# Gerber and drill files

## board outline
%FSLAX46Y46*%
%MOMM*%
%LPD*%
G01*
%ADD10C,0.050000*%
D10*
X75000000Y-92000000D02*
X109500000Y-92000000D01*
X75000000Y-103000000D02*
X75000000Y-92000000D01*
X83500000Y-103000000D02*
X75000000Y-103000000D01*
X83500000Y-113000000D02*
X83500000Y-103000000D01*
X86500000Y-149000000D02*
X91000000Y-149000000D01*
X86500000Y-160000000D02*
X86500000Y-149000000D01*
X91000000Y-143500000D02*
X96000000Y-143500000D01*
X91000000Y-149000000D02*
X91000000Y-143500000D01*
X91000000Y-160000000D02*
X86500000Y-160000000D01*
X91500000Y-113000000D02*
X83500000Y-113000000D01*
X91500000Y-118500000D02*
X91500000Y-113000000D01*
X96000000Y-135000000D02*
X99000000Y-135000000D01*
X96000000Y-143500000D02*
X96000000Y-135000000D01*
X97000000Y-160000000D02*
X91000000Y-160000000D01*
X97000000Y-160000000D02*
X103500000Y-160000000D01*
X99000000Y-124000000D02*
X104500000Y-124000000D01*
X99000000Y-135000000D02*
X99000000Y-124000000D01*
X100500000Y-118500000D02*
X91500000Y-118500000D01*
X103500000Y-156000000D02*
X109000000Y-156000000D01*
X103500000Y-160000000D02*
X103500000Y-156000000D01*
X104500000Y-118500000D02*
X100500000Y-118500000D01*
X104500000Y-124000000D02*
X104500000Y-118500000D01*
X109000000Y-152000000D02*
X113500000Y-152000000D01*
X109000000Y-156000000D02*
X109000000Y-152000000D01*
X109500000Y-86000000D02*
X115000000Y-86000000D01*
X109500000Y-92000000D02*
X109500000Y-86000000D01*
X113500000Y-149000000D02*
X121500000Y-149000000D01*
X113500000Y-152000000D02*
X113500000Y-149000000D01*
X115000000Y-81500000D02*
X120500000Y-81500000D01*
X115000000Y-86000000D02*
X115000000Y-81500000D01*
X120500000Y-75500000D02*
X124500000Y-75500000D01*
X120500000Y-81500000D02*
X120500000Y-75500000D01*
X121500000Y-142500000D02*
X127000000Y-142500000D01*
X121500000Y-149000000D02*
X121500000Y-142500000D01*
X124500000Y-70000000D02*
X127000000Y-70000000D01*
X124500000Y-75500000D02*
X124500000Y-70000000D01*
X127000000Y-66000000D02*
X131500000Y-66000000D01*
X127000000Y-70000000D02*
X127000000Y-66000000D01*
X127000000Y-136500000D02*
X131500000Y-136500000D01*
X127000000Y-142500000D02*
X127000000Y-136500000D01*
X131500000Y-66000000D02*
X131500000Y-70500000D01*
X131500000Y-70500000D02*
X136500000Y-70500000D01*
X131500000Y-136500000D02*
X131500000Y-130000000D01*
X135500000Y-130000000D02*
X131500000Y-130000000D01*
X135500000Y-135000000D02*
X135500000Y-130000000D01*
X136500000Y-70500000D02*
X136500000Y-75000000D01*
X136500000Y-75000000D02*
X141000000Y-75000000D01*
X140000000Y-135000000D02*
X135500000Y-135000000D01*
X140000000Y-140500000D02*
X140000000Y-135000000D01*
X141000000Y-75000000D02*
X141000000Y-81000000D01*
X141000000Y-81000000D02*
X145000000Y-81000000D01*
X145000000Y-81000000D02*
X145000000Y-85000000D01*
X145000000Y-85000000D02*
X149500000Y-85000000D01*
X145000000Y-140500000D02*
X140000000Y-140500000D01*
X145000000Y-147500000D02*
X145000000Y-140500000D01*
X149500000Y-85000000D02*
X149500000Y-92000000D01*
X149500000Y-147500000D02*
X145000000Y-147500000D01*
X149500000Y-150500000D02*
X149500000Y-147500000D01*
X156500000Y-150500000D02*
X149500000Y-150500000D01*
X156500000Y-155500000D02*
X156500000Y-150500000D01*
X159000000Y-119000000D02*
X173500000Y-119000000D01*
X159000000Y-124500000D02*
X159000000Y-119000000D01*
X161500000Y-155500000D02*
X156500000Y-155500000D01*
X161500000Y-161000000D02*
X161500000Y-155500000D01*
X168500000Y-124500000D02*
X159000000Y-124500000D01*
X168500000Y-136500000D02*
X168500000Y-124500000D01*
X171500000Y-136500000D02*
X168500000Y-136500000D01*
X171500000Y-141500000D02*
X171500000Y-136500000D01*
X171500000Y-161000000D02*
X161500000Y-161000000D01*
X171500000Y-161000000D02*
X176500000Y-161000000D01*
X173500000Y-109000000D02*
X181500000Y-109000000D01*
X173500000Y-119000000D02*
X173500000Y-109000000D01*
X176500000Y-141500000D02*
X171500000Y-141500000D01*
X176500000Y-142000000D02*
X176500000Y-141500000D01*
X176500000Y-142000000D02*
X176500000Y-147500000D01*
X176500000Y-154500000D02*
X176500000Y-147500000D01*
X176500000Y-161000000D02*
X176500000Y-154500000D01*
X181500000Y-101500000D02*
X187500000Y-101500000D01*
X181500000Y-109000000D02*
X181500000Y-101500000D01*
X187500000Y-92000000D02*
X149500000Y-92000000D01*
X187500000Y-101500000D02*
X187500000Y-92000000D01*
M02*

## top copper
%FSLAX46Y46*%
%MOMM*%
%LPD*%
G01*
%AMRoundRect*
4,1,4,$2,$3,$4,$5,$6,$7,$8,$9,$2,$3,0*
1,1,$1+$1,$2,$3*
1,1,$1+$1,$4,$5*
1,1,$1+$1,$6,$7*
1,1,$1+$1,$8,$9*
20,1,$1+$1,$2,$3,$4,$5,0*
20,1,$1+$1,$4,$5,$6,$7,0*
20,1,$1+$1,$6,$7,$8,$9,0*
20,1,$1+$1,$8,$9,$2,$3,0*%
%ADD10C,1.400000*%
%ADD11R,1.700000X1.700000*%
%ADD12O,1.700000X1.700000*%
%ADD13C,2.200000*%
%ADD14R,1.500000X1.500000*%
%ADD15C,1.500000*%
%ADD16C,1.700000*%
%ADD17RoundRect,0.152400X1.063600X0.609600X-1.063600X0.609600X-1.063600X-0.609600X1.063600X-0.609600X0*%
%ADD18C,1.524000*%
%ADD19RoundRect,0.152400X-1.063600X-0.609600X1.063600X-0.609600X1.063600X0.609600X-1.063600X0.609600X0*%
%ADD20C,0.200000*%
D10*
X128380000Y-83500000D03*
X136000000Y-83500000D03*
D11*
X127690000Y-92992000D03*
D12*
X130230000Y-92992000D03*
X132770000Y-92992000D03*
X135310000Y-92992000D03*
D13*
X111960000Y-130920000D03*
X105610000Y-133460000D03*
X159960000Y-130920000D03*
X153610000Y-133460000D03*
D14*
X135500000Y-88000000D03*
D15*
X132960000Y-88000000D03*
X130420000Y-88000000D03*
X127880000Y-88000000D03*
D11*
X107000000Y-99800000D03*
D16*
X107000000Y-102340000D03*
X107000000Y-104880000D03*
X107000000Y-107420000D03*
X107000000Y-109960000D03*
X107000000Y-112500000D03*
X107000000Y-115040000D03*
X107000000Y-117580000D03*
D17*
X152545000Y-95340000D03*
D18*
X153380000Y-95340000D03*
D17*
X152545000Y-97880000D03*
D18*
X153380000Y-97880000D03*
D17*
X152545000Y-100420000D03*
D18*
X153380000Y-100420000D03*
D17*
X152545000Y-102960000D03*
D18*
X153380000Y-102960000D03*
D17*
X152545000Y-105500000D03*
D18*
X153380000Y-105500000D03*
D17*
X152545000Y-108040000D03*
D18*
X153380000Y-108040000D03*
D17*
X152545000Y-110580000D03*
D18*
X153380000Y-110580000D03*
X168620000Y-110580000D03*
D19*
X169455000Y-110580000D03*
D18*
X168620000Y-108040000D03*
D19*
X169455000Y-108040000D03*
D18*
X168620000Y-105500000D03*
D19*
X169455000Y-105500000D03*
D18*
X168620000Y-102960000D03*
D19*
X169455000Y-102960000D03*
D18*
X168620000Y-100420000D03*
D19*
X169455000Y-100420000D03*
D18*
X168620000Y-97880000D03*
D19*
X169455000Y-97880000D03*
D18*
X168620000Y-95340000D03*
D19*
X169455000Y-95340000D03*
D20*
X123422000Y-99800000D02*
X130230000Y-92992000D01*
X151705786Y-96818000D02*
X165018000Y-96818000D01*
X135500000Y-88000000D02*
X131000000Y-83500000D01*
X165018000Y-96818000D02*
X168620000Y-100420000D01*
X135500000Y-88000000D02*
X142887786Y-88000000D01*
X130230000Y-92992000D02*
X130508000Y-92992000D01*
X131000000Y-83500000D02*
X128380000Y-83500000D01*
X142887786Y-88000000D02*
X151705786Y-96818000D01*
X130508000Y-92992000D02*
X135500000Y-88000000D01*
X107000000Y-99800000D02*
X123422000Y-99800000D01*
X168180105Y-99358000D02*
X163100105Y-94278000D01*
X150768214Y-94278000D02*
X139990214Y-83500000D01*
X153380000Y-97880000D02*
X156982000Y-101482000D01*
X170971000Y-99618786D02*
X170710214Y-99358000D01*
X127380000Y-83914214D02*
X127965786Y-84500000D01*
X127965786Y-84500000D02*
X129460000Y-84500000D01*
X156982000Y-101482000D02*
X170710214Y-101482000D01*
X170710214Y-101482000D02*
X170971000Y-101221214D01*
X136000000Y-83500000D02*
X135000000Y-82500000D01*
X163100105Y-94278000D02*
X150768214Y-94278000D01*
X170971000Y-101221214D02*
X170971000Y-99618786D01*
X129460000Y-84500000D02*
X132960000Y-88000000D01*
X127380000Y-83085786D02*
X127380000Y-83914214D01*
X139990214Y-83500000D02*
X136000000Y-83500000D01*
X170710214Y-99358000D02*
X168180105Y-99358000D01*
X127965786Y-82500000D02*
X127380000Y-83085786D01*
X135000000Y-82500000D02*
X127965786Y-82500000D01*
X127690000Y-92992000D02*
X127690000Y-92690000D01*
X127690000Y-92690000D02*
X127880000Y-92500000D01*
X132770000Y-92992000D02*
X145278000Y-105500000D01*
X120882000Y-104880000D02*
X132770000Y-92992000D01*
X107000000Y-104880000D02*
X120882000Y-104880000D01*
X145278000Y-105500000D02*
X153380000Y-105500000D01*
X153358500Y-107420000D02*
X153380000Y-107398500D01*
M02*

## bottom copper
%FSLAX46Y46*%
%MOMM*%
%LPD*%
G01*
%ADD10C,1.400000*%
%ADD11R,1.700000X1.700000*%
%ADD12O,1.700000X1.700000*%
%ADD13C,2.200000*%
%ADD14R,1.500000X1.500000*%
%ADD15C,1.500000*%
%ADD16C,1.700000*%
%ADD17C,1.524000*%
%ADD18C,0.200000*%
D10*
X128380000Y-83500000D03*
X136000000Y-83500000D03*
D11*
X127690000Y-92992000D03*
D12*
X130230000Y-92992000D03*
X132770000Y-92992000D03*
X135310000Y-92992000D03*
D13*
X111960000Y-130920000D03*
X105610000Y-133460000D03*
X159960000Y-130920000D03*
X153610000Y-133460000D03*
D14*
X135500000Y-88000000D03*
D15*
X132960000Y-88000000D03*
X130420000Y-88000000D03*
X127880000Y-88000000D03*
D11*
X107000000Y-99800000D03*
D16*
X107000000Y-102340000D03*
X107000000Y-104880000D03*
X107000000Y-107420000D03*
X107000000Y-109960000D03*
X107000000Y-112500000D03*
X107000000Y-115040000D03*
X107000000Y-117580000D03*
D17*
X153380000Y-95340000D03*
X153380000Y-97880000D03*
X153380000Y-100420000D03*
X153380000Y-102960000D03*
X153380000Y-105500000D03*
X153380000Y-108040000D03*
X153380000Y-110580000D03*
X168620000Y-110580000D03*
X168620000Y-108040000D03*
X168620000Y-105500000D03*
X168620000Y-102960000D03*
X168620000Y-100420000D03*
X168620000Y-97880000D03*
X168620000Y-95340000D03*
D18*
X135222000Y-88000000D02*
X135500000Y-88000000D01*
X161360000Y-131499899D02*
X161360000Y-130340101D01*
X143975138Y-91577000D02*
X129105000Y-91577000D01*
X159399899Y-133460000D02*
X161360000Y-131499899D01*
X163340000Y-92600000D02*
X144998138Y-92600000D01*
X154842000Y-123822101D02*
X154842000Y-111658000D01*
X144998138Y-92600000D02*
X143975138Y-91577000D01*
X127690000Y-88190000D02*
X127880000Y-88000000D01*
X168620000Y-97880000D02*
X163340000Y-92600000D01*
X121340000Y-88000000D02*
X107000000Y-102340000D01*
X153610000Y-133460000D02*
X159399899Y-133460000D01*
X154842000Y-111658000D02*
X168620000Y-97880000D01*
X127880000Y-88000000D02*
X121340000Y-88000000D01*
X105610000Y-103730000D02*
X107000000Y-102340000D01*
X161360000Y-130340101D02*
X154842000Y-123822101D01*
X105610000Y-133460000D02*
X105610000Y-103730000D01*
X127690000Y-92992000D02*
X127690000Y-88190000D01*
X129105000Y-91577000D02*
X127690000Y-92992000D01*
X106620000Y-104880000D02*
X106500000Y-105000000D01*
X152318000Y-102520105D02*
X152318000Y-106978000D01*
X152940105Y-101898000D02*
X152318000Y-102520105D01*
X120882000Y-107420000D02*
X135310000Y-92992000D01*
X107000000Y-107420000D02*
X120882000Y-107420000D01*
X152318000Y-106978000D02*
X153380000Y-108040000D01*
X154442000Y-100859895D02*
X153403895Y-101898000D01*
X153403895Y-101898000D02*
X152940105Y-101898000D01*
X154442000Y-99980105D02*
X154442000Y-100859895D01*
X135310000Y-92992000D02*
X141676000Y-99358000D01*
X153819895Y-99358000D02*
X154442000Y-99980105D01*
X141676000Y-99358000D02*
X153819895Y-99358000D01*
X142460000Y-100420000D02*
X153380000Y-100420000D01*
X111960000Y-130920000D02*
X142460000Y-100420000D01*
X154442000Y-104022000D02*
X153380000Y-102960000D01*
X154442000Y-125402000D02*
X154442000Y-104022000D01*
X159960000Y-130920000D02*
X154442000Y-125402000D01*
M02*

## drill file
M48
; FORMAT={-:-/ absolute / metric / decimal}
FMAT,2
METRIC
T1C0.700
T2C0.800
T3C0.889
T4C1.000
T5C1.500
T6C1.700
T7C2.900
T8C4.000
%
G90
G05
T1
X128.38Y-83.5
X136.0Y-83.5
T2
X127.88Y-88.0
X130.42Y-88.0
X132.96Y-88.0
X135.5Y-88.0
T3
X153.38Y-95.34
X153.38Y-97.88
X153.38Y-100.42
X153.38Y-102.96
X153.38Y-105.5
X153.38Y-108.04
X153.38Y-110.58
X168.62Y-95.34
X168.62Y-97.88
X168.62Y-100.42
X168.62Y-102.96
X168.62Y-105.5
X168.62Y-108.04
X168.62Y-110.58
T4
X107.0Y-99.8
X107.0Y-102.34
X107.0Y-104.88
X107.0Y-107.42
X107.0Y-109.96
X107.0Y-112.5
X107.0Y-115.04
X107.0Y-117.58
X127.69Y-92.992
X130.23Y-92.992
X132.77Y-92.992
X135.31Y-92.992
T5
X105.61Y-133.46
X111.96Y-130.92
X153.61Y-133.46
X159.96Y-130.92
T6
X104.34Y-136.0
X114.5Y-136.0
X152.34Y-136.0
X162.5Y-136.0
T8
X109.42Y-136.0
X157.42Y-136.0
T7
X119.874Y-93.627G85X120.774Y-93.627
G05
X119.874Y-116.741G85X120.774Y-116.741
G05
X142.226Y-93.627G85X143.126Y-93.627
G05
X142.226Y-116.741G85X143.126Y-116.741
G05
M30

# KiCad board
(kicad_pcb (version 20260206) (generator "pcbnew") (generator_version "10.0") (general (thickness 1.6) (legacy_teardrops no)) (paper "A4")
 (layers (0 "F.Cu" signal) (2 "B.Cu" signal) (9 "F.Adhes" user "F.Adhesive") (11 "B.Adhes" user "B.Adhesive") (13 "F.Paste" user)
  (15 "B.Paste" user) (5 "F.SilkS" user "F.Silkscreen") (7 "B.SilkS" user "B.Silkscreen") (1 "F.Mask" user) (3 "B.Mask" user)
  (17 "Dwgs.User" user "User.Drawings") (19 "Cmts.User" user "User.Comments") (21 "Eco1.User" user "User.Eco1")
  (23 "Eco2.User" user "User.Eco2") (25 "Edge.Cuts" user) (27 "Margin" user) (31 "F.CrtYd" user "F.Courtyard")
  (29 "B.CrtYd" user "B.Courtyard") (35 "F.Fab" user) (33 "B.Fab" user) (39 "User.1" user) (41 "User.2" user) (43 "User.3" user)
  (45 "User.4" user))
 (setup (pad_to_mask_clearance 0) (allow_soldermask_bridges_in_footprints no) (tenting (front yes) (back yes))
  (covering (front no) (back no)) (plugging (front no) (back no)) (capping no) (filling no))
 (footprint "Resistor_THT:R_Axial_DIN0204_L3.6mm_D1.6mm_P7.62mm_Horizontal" (layer "F.Cu") (at 128.38 83.5)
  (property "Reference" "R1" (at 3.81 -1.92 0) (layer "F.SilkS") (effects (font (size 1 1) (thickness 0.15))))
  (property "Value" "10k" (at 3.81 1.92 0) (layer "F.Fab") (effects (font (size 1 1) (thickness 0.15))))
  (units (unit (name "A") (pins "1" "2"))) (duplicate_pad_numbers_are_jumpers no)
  (pad "1" thru_hole circle (at 0 0) (size 1.4 1.4) (drill 0.7) (layers "*.Cu" "*.Mask") (remove_unused_layers no) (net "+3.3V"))
  (pad "2" thru_hole circle (at 7.62 0) (size 1.4 1.4) (drill 0.7) (layers "*.Cu" "*.Mask") (remove_unused_layers no) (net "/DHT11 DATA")))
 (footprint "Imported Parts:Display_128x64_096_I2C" (layer "F.Cu") (at 131.5 92.992)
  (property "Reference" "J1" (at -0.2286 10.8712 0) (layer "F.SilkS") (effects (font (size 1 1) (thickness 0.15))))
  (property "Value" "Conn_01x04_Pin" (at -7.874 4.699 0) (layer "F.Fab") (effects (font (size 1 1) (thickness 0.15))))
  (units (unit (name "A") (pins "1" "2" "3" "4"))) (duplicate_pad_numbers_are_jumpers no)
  (pad "" np_thru_hole oval (at -11.176 0.635) (size 3.8 2.9) (drill oval 3.8 2.9) (layers "*.Cu" "*.Mask"))
  (pad "" np_thru_hole oval (at -11.176 23.749) (size 3.8 2.9) (drill oval 3.8 2.9) (layers "*.Cu" "*.Mask"))
  (pad "" np_thru_hole oval (at 11.176 0.635) (size 3.8 2.9) (drill oval 3.8 2.9) (layers "*.Cu" "*.Mask"))
  (pad "" np_thru_hole oval (at 11.176 23.749) (size 3.8 2.9) (drill oval 3.8 2.9) (layers "*.Cu" "*.Mask"))
  (pad "1" thru_hole rect (at -3.81 0 90) (size 1.7 1.7) (drill 1) (layers "*.Cu" "*.Mask") (remove_unused_layers no) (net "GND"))
  (pad "2" thru_hole oval (at -1.27 0 90) (size 1.7 1.7) (drill 1) (layers "*.Cu" "*.Mask") (remove_unused_layers no) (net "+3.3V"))
  (pad "3" thru_hole oval (at 1.27 0 90) (size 1.7 1.7) (drill 1) (layers "*.Cu" "*.Mask") (remove_unused_layers no) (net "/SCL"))
  (pad "4" thru_hole oval (at 3.81 0 90) (size 1.7 1.7) (drill 1) (layers "*.Cu" "*.Mask") (remove_unused_layers no) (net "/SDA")))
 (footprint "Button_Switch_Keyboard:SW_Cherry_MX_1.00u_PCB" (layer "F.Cu") (at 111.96 130.92)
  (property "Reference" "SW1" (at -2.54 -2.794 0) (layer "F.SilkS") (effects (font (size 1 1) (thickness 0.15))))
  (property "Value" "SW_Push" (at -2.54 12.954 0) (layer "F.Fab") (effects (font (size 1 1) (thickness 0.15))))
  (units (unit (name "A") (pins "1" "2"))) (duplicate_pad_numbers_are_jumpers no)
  (pad "" np_thru_hole circle (at -7.62 5.08) (size 1.7 1.7) (drill 1.7) (layers "*.Cu" "*.Mask"))
  (pad "" np_thru_hole circle (at -2.54 5.08) (size 4 4) (drill 4) (layers "*.Cu" "*.Mask"))
  (pad "" np_thru_hole circle (at 2.54 5.08) (size 1.7 1.7) (drill 1.7) (layers "*.Cu" "*.Mask"))
  (pad "1" thru_hole circle (at 0 0) (size 2.2 2.2) (drill 1.5) (layers "*.Cu" "*.Mask") (remove_unused_layers no) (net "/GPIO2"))
  (pad "2" thru_hole circle (at -6.35 2.54) (size 2.2 2.2) (drill 1.5) (layers "*.Cu" "*.Mask") (remove_unused_layers no) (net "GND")))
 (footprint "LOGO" (layer "F.Cu") (at 132.984888 107.481245)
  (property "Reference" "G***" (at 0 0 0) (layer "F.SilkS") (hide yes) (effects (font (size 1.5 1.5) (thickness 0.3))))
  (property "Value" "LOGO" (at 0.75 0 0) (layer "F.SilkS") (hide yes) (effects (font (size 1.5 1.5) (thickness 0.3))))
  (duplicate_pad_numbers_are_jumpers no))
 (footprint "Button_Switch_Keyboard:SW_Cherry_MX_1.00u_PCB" (layer "F.Cu") (at 159.96 130.92)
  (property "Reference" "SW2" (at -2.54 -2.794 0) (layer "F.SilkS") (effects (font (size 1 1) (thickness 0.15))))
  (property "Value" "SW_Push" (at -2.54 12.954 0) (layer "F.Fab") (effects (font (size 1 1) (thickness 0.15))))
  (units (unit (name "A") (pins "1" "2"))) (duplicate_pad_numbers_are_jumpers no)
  (pad "" np_thru_hole circle (at -7.62 5.08) (size 1.7 1.7) (drill 1.7) (layers "*.Cu" "*.Mask"))
  (pad "" np_thru_hole circle (at -2.54 5.08) (size 4 4) (drill 4) (layers "*.Cu" "*.Mask"))
  (pad "" np_thru_hole circle (at 2.54 5.08) (size 1.7 1.7) (drill 1.7) (layers "*.Cu" "*.Mask"))
  (pad "1" thru_hole circle (at 0 0) (size 2.2 2.2) (drill 1.5) (layers "*.Cu" "*.Mask") (remove_unused_layers no) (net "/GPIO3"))
  (pad "2" thru_hole circle (at -6.35 2.54) (size 2.2 2.2) (drill 1.5) (layers "*.Cu" "*.Mask") (remove_unused_layers no) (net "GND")))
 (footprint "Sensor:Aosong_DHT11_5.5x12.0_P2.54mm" (layer "F.Cu") (at 135.5 88 -90)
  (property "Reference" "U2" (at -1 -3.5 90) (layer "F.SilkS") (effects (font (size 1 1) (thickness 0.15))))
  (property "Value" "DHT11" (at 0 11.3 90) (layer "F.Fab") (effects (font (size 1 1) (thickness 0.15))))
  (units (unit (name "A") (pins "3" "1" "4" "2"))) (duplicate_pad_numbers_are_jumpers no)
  (pad "1" thru_hole rect (at 0 0 270) (size 1.5 1.5) (drill 0.8) (layers "*.Cu" "*.Mask") (remove_unused_layers no) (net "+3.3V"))
  (pad "2" thru_hole circle (at 0 2.54 270) (size 1.5 1.5) (drill 0.8) (layers "*.Cu" "*.Mask") (remove_unused_layers no)
   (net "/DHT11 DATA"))
  (pad "3" thru_hole circle (at 0 5.08 270) (size 1.5 1.5) (drill 0.8) (layers "*.Cu" "*.Mask") (remove_unused_layers no)
   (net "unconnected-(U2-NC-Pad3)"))
  (pad "4" thru_hole circle (at 0 7.62 270) (size 1.5 1.5) (drill 0.8) (layers "*.Cu" "*.Mask") (remove_unused_layers no) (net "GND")))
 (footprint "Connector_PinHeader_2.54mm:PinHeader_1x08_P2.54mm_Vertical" (layer "F.Cu") (at 107 99.8)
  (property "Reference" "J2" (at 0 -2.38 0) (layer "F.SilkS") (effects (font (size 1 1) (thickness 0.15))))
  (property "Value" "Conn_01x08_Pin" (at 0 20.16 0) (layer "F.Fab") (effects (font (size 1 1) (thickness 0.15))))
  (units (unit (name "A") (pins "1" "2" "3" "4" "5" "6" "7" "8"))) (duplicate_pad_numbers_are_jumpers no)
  (pad "1" thru_hole rect (at 0 0) (size 1.7 1.7) (drill 1) (layers "*.Cu" "*.Mask") (remove_unused_layers no) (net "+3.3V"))
  (pad "2" thru_hole circle (at 0 2.54) (size 1.7 1.7) (drill 1) (layers "*.Cu" "*.Mask") (remove_unused_layers no) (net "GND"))
  (pad "3" thru_hole circle (at 0 5.08) (size 1.7 1.7) (drill 1) (layers "*.Cu" "*.Mask") (remove_unused_layers no) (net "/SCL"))
  (pad "4" thru_hole circle (at 0 7.62) (size 1.7 1.7) (drill 1) (layers "*.Cu" "*.Mask") (remove_unused_layers no) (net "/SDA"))
  (pad "5" thru_hole circle (at 0 10.16) (size 1.7 1.7) (drill 1) (layers "*.Cu" "*.Mask") (remove_unused_layers no)
   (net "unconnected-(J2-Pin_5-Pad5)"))
  (pad "6" thru_hole circle (at 0 12.7) (size 1.7 1.7) (drill 1) (layers "*.Cu" "*.Mask") (remove_unused_layers no)
   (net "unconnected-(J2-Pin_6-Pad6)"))
  (pad "7" thru_hole circle (at 0 15.24) (size 1.7 1.7) (drill 1) (layers "*.Cu" "*.Mask") (remove_unused_layers no)
   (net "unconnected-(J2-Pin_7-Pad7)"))
  (pad "8" thru_hole circle (at 0 17.78) (size 1.7 1.7) (drill 1) (layers "*.Cu" "*.Mask") (remove_unused_layers no)
   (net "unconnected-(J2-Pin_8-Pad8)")))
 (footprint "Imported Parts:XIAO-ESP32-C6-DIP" (layer "F.Cu") (at 161 102.96 90)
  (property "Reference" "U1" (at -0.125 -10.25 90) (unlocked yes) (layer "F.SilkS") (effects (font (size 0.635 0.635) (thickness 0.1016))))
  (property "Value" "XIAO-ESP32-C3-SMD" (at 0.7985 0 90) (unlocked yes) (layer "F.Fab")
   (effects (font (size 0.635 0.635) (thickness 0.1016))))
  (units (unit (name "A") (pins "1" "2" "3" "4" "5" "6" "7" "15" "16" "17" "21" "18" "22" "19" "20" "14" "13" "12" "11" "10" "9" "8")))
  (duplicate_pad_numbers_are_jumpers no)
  (pad "1" smd roundrect (at 7.62 -8.455 180) (size 2.432 1.524) (layers "F.Cu" "F.Mask") (roundrect_rratio 0.1)
   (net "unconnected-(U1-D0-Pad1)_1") (thermal_bridge_angle 45))
  (pad "1" thru_hole circle (at 7.62 -7.62 180) (size 1.524 1.524) (drill 0.889) (layers "*.Cu" "*.Mask") (remove_unused_layers no)
   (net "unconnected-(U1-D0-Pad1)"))
  (pad "2" smd roundrect (at 5.08 -8.455 180) (size 2.432 1.524) (layers "F.Cu" "F.Mask") (roundrect_rratio 0.1) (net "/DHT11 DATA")
   (thermal_bridge_angle 45))
  (pad "2" thru_hole circle (at 5.08 -7.62 180) (size 1.524 1.524) (drill 0.889) (layers "*.Cu" "*.Mask") (remove_unused_layers no)
   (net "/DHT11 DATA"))
  (pad "3" smd roundrect (at 2.54 -8.455 180) (size 2.432 1.524) (layers "F.Cu" "F.Mask") (roundrect_rratio 0.1) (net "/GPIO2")
   (thermal_bridge_angle 45))
  (pad "3" thru_hole circle (at 2.54 -7.62 180) (size 1.524 1.524) (drill 0.889) (layers "*.Cu" "*.Mask") (remove_unused_layers no)
   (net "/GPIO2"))
  (pad "4" smd roundrect (at 0 -8.455 180) (size 2.432 1.524) (layers "F.Cu" "F.Mask") (roundrect_rratio 0.1) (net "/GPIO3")
   (thermal_bridge_angle 45))
  (pad "4" thru_hole circle (at 0 -7.62 180) (size 1.524 1.524) (drill 0.889) (layers "*.Cu" "*.Mask") (remove_unused_layers no)
   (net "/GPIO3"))
  (pad "5" smd roundrect (at -2.54 -8.455 180) (size 2.432 1.524) (layers "F.Cu" "F.Mask") (roundrect_rratio 0.1) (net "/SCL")
   (thermal_bridge_angle 45))
  (pad "5" thru_hole circle (at -2.54 -7.62 180) (size 1.524 1.524) (drill 0.889) (layers "*.Cu" "*.Mask") (remove_unused_layers no)
   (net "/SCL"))
  (pad "6" smd roundrect (at -5.08 -8.455 180) (size 2.432 1.524) (layers "F.Cu" "F.Mask") (roundrect_rratio 0.1) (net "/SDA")
   (thermal_bridge_angle 45))
  (pad "6" thru_hole circle (at -5.08 -7.62 180) (size 1.524 1.524) (drill 0.889) (layers "*.Cu" "*.Mask") (remove_unused_layers no)
   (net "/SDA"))
  (pad "7" smd roundrect (at -7.62 -8.455 180) (size 2.432 1.524) (layers "F.Cu" "F.Mask") (roundrect_rratio 0.1)
   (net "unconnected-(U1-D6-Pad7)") (thermal_bridge_angle 45))
  (pad "7" thru_hole circle (at -7.62 -7.62 180) (size 1.524 1.524) (drill 0.889) (layers "*.Cu" "*.Mask") (remove_unused_layers no)
   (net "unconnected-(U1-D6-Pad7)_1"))
  (pad "8" thru_hole circle (at -7.62 7.62) (size 1.524 1.524) (drill 0.889) (layers "*.Cu" "*.Mask") (remove_unused_layers no)
   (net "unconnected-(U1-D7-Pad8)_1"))
  (pad "8" smd roundrect (at -7.62 8.455) (size 2.432 1.524) (layers "F.Cu" "F.Mask") (roundrect_rratio 0.1)
   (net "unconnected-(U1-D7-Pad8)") (thermal_bridge_angle 45))
  (pad "9" thru_hole circle (at -5.08 7.62) (size 1.524 1.524) (drill 0.889) (layers "*.Cu" "*.Mask") (remove_unused_layers no)
   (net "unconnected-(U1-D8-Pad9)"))
  (pad "9" smd roundrect (at -5.08 8.455) (size 2.432 1.524) (layers "F.Cu" "F.Mask") (roundrect_rratio 0.1)
   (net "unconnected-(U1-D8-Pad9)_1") (thermal_bridge_angle 45))
  (pad "10" thru_hole circle (at -2.54 7.62) (size 1.524 1.524) (drill 0.889) (layers "*.Cu" "*.Mask") (remove_unused_layers no)
   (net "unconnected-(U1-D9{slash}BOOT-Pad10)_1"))
  (pad "10" smd roundrect (at -2.54 8.455) (size 2.432 1.524) (layers "F.Cu" "F.Mask") (roundrect_rratio 0.1)
   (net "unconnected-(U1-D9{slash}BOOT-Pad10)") (thermal_bridge_angle 45))
  (pad "11" thru_hole circle (at 0 7.62) (size 1.524 1.524) (drill 0.889) (layers "*.Cu" "*.Mask") (remove_unused_layers no)
   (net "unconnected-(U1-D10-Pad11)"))
  (pad "11" smd roundrect (at 0 8.455) (size 2.432 1.524) (layers "F.Cu" "F.Mask") (roundrect_rratio 0.1)
   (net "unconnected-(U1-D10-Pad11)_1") (thermal_bridge_angle 45))
  (pad "12" thru_hole circle (at 2.54 7.62) (size 1.524 1.524) (drill 0.889) (layers "*.Cu" "*.Mask") (remove_unused_layers no)
   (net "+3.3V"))
  (pad "12" smd roundrect (at 2.54 8.455) (size 2.432 1.524) (layers "F.Cu" "F.Mask") (roundrect_rratio 0.1) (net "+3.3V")
   (thermal_bridge_angle 45))
  (pad "13" thru_hole circle (at 5.08 7.62) (size 1.524 1.524) (drill 0.889) (layers "*.Cu" "*.Mask") (remove_unused_layers no) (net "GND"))
  (pad "13" smd roundrect (at 5.08 8.455) (size 2.432 1.524) (layers "F.Cu" "F.Mask") (roundrect_rratio 0.1) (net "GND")
   (thermal_bridge_angle 45))
  (pad "14" thru_hole circle (at 7.62 7.62) (size 1.524 1.524) (drill 0.889) (layers "*.Cu" "*.Mask") (remove_unused_layers no) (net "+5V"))
  (pad "14" smd roundrect (at 7.62 8.455) (size 2.432 1.524) (layers "F.Cu" "F.Mask") (roundrect_rratio 0.1) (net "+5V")
   (thermal_bridge_angle 45)))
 (gr_line (start 75 92) (end 109.5 92) (stroke (width 0.05) (type default)) (layer "Edge.Cuts"))
 (gr_line (start 75 103) (end 75 92) (stroke (width 0.05) (type default)) (layer "Edge.Cuts"))
 (gr_line (start 83.5 103) (end 75 103) (stroke (width 0.05) (type default)) (layer "Edge.Cuts"))
 (gr_line (start 83.5 113) (end 83.5 103) (stroke (width 0.05) (type default)) (layer "Edge.Cuts"))
 (gr_line (start 86.5 149) (end 91 149) (stroke (width 0.05) (type default)) (layer "Edge.Cuts"))
 (gr_line (start 86.5 160) (end 86.5 149) (stroke (width 0.05) (type default)) (layer "Edge.Cuts"))
 (gr_line (start 91 143.5) (end 96 143.5) (stroke (width 0.05) (type default)) (layer "Edge.Cuts"))
 (gr_line (start 91 149) (end 91 143.5) (stroke (width 0.05) (type default)) (layer "Edge.Cuts"))
 (gr_line (start 91 160) (end 86.5 160) (stroke (width 0.05) (type default)) (layer "Edge.Cuts"))
 (gr_line (start 91.5 113) (end 83.5 113) (stroke (width 0.05) (type default)) (layer "Edge.Cuts"))
 (gr_line (start 91.5 118.5) (end 91.5 113) (stroke (width 0.05) (type default)) (layer "Edge.Cuts"))
 (gr_line (start 96 135) (end 99 135) (stroke (width 0.05) (type default)) (layer "Edge.Cuts"))
 (gr_line (start 96 143.5) (end 96 135) (stroke (width 0.05) (type default)) (layer "Edge.Cuts"))
 (gr_line (start 97 160) (end 91 160) (stroke (width 0.05) (type default)) (layer "Edge.Cuts"))
 (gr_line (start 97 160) (end 103.5 160) (stroke (width 0.05) (type default)) (layer "Edge.Cuts"))
 (gr_line (start 99 124) (end 104.5 124) (stroke (width 0.05) (type default)) (layer "Edge.Cuts"))
 (gr_line (start 99 135) (end 99 124) (stroke (width 0.05) (type default)) (layer "Edge.Cuts"))
 (gr_line (start 100.5 118.5) (end 91.5 118.5) (stroke (width 0.05) (type default)) (layer "Edge.Cuts"))
 (gr_line (start 103.5 156) (end 109 156) (stroke (width 0.05) (type default)) (layer "Edge.Cuts"))
 (gr_line (start 103.5 160) (end 103.5 156) (stroke (width 0.05) (type default)) (layer "Edge.Cuts"))
 (gr_line (start 104.5 118.5) (end 100.5 118.5) (stroke (width 0.05) (type default)) (layer "Edge.Cuts"))
 (gr_line (start 104.5 124) (end 104.5 118.5) (stroke (width 0.05) (type default)) (layer "Edge.Cuts"))
 (gr_line (start 109 152) (end 113.5 152) (stroke (width 0.05) (type default)) (layer "Edge.Cuts"))
 (gr_line (start 109 156) (end 109 152) (stroke (width 0.05) (type default)) (layer "Edge.Cuts"))
 (gr_line (start 109.5 86) (end 115 86) (stroke (width 0.05) (type default)) (layer "Edge.Cuts"))
 (gr_line (start 109.5 92) (end 109.5 86) (stroke (width 0.05) (type default)) (layer "Edge.Cuts"))
 (gr_line (start 113.5 149) (end 121.5 149) (stroke (width 0.05) (type default)) (layer "Edge.Cuts"))
 (gr_line (start 113.5 152) (end 113.5 149) (stroke (width 0.05) (type default)) (layer "Edge.Cuts"))
 (gr_line (start 115 81.5) (end 120.5 81.5) (stroke (width 0.05) (type default)) (layer "Edge.Cuts"))
 (gr_line (start 115 86) (end 115 81.5) (stroke (width 0.05) (type default)) (layer "Edge.Cuts"))
 (gr_line (start 120.5 75.5) (end 124.5 75.5) (stroke (width 0.05) (type default)) (layer "Edge.Cuts"))
 (gr_line (start 120.5 81.5) (end 120.5 75.5) (stroke (width 0.05) (type default)) (layer "Edge.Cuts"))
 (gr_line (start 121.5 142.5) (end 127 142.5) (stroke (width 0.05) (type default)) (layer "Edge.Cuts"))
 (gr_line (start 121.5 149) (end 121.5 142.5) (stroke (width 0.05) (type default)) (layer "Edge.Cuts"))
 (gr_line (start 124.5 70) (end 127 70) (stroke (width 0.05) (type default)) (layer "Edge.Cuts"))
 (gr_line (start 124.5 75.5) (end 124.5 70) (stroke (width 0.05) (type default)) (layer "Edge.Cuts"))
 (gr_line (start 127 66) (end 131.5 66) (stroke (width 0.05) (type default)) (layer "Edge.Cuts"))
 (gr_line (start 127 70) (end 127 66) (stroke (width 0.05) (type default)) (layer "Edge.Cuts"))
 (gr_line (start 127 136.5) (end 131.5 136.5) (stroke (width 0.05) (type default)) (layer "Edge.Cuts"))
 (gr_line (start 127 142.5) (end 127 136.5) (stroke (width 0.05) (type default)) (layer "Edge.Cuts"))
 (gr_line (start 131.5 66) (end 131.5 70.5) (stroke (width 0.05) (type default)) (layer "Edge.Cuts"))
 (gr_line (start 131.5 70.5) (end 136.5 70.5) (stroke (width 0.05) (type default)) (layer "Edge.Cuts"))
 (gr_line (start 131.5 136.5) (end 131.5 130) (stroke (width 0.05) (type default)) (layer "Edge.Cuts"))
 (gr_line (start 135.5 130) (end 131.5 130) (stroke (width 0.05) (type default)) (layer "Edge.Cuts"))
 (gr_line (start 135.5 135) (end 135.5 130) (stroke (width 0.05) (type default)) (layer "Edge.Cuts"))
 (gr_line (start 136.5 70.5) (end 136.5 75) (stroke (width 0.05) (type default)) (layer "Edge.Cuts"))
 (gr_line (start 136.5 75) (end 141 75) (stroke (width 0.05) (type default)) (layer "Edge.Cuts"))
 (gr_line (start 140 135) (end 135.5 135) (stroke (width 0.05) (type default)) (layer "Edge.Cuts"))
 (gr_line (start 140 140.5) (end 140 135) (stroke (width 0.05) (type default)) (layer "Edge.Cuts"))
 (gr_line (start 141 75) (end 141 81) (stroke (width 0.05) (type default)) (layer "Edge.Cuts"))
 (gr_line (start 141 81) (end 145 81) (stroke (width 0.05) (type default)) (layer "Edge.Cuts"))
 (gr_line (start 145 81) (end 145 85) (stroke (width 0.05) (type default)) (layer "Edge.Cuts"))
 (gr_line (start 145 85) (end 149.5 85) (stroke (width 0.05) (type default)) (layer "Edge.Cuts"))
 (gr_line (start 145 140.5) (end 140 140.5) (stroke (width 0.05) (type default)) (layer "Edge.Cuts"))
 (gr_line (start 145 147.5) (end 145 140.5) (stroke (width 0.05) (type default)) (layer "Edge.Cuts"))
 (gr_line (start 149.5 85) (end 149.5 92) (stroke (width 0.05) (type default)) (layer "Edge.Cuts"))
 (gr_line (start 149.5 147.5) (end 145 147.5) (stroke (width 0.05) (type default)) (layer "Edge.Cuts"))
 (gr_line (start 149.5 150.5) (end 149.5 147.5) (stroke (width 0.05) (type default)) (layer "Edge.Cuts"))
 (gr_line (start 156.5 150.5) (end 149.5 150.5) (stroke (width 0.05) (type default)) (layer "Edge.Cuts"))
 (gr_line (start 156.5 155.5) (end 156.5 150.5) (stroke (width 0.05) (type default)) (layer "Edge.Cuts"))
 (gr_line (start 159 119) (end 173.5 119) (stroke (width 0.05) (type default)) (layer "Edge.Cuts"))
 (gr_line (start 159 124.5) (end 159 119) (stroke (width 0.05) (type default)) (layer "Edge.Cuts"))
 (gr_line (start 161.5 155.5) (end 156.5 155.5) (stroke (width 0.05) (type default)) (layer "Edge.Cuts"))
 (gr_line (start 161.5 161) (end 161.5 155.5) (stroke (width 0.05) (type default)) (layer "Edge.Cuts"))
 (gr_line (start 168.5 124.5) (end 159 124.5) (stroke (width 0.05) (type default)) (layer "Edge.Cuts"))
 (gr_line (start 168.5 136.5) (end 168.5 124.5) (stroke (width 0.05) (type default)) (layer "Edge.Cuts"))
 (gr_line (start 171.5 136.5) (end 168.5 136.5) (stroke (width 0.05) (type default)) (layer "Edge.Cuts"))
 (gr_line (start 171.5 141.5) (end 171.5 136.5) (stroke (width 0.05) (type default)) (layer "Edge.Cuts"))
 (gr_line (start 171.5 161) (end 161.5 161) (stroke (width 0.05) (type default)) (layer "Edge.Cuts"))
 (gr_line (start 171.5 161) (end 176.5 161) (stroke (width 0.05) (type default)) (layer "Edge.Cuts"))
 (gr_line (start 173.5 109) (end 181.5 109) (stroke (width 0.05) (type default)) (layer "Edge.Cuts"))
 (gr_line (start 173.5 119) (end 173.5 109) (stroke (width 0.05) (type default)) (layer "Edge.Cuts"))
 (gr_line (start 176.5 141.5) (end 171.5 141.5) (stroke (width 0.05) (type default)) (layer "Edge.Cuts"))
 (gr_line (start 176.5 142) (end 176.5 141.5) (stroke (width 0.05) (type default)) (layer "Edge.Cuts"))
 (gr_line (start 176.5 142) (end 176.5 147.5) (stroke (width 0.05) (type default)) (layer "Edge.Cuts"))
 (gr_line (start 176.5 154.5) (end 176.5 147.5) (stroke (width 0.05) (type default)) (layer "Edge.Cuts"))
 (gr_line (start 176.5 161) (end 176.5 154.5) (stroke (width 0.05) (type default)) (layer "Edge.Cuts"))
 (gr_line (start 181.5 101.5) (end 187.5 101.5) (stroke (width 0.05) (type default)) (layer "Edge.Cuts"))
 (gr_line (start 181.5 109) (end 181.5 101.5) (stroke (width 0.05) (type default)) (layer "Edge.Cuts"))
 (gr_line (start 187.5 92) (end 149.5 92) (stroke (width 0.05) (type default)) (layer "Edge.Cuts"))
 (gr_line (start 187.5 101.5) (end 187.5 92) (stroke (width 0.05) (type default)) (layer "Edge.Cuts"))
 (segment (start 123.422 99.8) (end 130.23 92.992) (width 0.2) (layer "F.Cu") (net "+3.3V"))
 (segment (start 151.705786 96.818) (end 165.018 96.818) (width 0.2) (layer "F.Cu") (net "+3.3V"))
 (segment (start 135.5 88) (end 131 83.5) (width 0.2) (layer "F.Cu") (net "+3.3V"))
 (segment (start 165.018 96.818) (end 168.62 100.42) (width 0.2) (layer "F.Cu") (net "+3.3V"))
 (segment (start 135.5 88) (end 142.887786 88) (width 0.2) (layer "F.Cu") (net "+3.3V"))
 (segment (start 130.23 92.992) (end 130.508 92.992) (width 0.2) (layer "F.Cu") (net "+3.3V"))
 (segment (start 131 83.5) (end 128.38 83.5) (width 0.2) (layer "F.Cu") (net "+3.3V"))
 (segment (start 142.887786 88) (end 151.705786 96.818) (width 0.2) (layer "F.Cu") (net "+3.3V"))
 (segment (start 130.508 92.992) (end 135.5 88) (width 0.2) (layer "F.Cu") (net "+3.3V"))
 (segment (start 107 99.8) (end 123.422 99.8) (width 0.2) (layer "F.Cu") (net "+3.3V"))
 (segment (start 135.222 88) (end 135.5 88) (width 0.2) (layer "B.Cu") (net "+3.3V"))
 (segment (start 168.180105 99.358) (end 163.100105 94.278) (width 0.2) (layer "F.Cu") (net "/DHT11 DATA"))
 (segment (start 150.768214 94.278) (end 139.990214 83.5) (width 0.2) (layer "F.Cu") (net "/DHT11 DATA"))
 (segment (start 153.38 97.88) (end 156.982 101.482) (width 0.2) (layer "F.Cu") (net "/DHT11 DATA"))
 (segment (start 170.971 99.618786) (end 170.710214 99.358) (width 0.2) (layer "F.Cu") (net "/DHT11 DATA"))
 (segment (start 127.38 83.914214) (end 127.965786 84.5) (width 0.2) (layer "F.Cu") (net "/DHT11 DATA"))
 (segment (start 127.965786 84.5) (end 129.46 84.5) (width 0.2) (layer "F.Cu") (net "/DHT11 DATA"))
 (segment (start 156.982 101.482) (end 170.710214 101.482) (width 0.2) (layer "F.Cu") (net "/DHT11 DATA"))
 (segment (start 170.710214 101.482) (end 170.971 101.221214) (width 0.2) (layer "F.Cu") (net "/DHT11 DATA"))
 (segment (start 136 83.5) (end 135 82.5) (width 0.2) (layer "F.Cu") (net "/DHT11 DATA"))
 (segment (start 163.100105 94.278) (end 150.768214 94.278) (width 0.2) (layer "F.Cu") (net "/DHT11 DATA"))
 (segment (start 170.971 101.221214) (end 170.971 99.618786) (width 0.2) (layer "F.Cu") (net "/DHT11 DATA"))
 (segment (start 129.46 84.5) (end 132.96 88) (width 0.2) (layer "F.Cu") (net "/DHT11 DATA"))
 (segment (start 127.38 83.085786) (end 127.38 83.914214) (width 0.2) (layer "F.Cu") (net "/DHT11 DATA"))
 (segment (start 139.990214 83.5) (end 136 83.5) (width 0.2) (layer "F.Cu") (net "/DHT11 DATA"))
 (segment (start 170.710214 99.358) (end 168.180105 99.358) (width 0.2) (layer "F.Cu") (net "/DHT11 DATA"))
 (segment (start 127.965786 82.5) (end 127.38 83.085786) (width 0.2) (layer "F.Cu") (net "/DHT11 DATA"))
 (segment (start 135 82.5) (end 127.965786 82.5) (width 0.2) (layer "F.Cu") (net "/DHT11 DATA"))
 (segment (start 127.69 92.992) (end 127.69 92.69) (width 0.2) (layer "F.Cu") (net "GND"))
 (segment (start 127.69 92.69) (end 127.88 92.5) (width 0.2) (layer "F.Cu") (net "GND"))
 (segment (start 161.36 131.499899) (end 161.36 130.340101) (width 0.2) (layer "B.Cu") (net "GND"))
 (segment (start 143.975138 91.577) (end 129.105 91.577) (width 0.2) (layer "B.Cu") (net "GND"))
 (segment (start 159.399899 133.46) (end 161.36 131.499899) (width 0.2) (layer "B.Cu") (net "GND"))
 (segment (start 163.34 92.6) (end 144.998138 92.6) (width 0.2) (layer "B.Cu") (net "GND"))
 (segment (start 154.842 123.822101) (end 154.842 111.658) (width 0.2) (layer "B.Cu") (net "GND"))
 (segment (start 144.998138 92.6) (end 143.975138 91.577) (width 0.2) (layer "B.Cu") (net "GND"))
 (segment (start 127.69 88.19) (end 127.88 88) (width 0.2) (layer "B.Cu") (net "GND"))
 (segment (start 168.62 97.88) (end 163.34 92.6) (width 0.2) (layer "B.Cu") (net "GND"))
 (segment (start 121.34 88) (end 107 102.34) (width 0.2) (layer "B.Cu") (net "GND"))
 (segment (start 153.61 133.46) (end 159.399899 133.46) (width 0.2) (layer "B.Cu") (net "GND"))
 (segment (start 154.842 111.658) (end 168.62 97.88) (width 0.2) (layer "B.Cu") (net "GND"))
 (segment (start 127.88 88) (end 121.34 88) (width 0.2) (layer "B.Cu") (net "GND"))
 (segment (start 105.61 103.73) (end 107 102.34) (width 0.2) (layer "B.Cu") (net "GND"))
 (segment (start 161.36 130.340101) (end 154.842 123.822101) (width 0.2) (layer "B.Cu") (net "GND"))
 (segment (start 105.61 133.46) (end 105.61 103.73) (width 0.2) (layer "B.Cu") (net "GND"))
 (segment (start 127.69 92.992) (end 127.69 88.19) (width 0.2) (layer "B.Cu") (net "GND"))
 (segment (start 129.105 91.577) (end 127.69 92.992) (width 0.2) (layer "B.Cu") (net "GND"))
 (segment (start 132.77 92.992) (end 145.278 105.5) (width 0.2) (layer "F.Cu") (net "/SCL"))
 (segment (start 120.882 104.88) (end 132.77 92.992) (width 0.2) (layer "F.Cu") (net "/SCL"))
 (segment (start 107 104.88) (end 120.882 104.88) (width 0.2) (layer "F.Cu") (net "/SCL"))
 (segment (start 145.278 105.5) (end 153.38 105.5) (width 0.2) (layer "F.Cu") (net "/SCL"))
 (segment (start 106.62 104.88) (end 106.5 105) (width 0.2) (layer "B.Cu") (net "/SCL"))
 (segment (start 153.3585 107.42) (end 153.38 107.3985) (width 0.2) (layer "F.Cu") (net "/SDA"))
 (segment (start 152.318 102.520105) (end 152.318 106.978) (width 0.2) (layer "B.Cu") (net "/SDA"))
 (segment (start 152.940105 101.898) (end 152.318 102.520105) (width 0.2) (layer "B.Cu") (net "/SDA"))
 (segment (start 120.882 107.42) (end 135.31 92.992) (width 0.2) (layer "B.Cu") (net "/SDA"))
 (segment (start 107 107.42) (end 120.882 107.42) (width 0.2) (layer "B.Cu") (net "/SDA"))
 (segment (start 152.318 106.978) (end 153.38 108.04) (width 0.2) (layer "B.Cu") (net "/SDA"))
 (segment (start 154.442 100.859895) (end 153.403895 101.898) (width 0.2) (layer "B.Cu") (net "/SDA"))
 (segment (start 153.403895 101.898) (end 152.940105 101.898) (width 0.2) (layer "B.Cu") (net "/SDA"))
 (segment (start 154.442 99.980105) (end 154.442 100.859895) (width 0.2) (layer "B.Cu") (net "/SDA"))
 (segment (start 135.31 92.992) (end 141.676 99.358) (width 0.2) (layer "B.Cu") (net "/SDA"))
 (segment (start 153.819895 99.358) (end 154.442 99.980105) (width 0.2) (layer "B.Cu") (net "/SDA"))
 (segment (start 141.676 99.358) (end 153.819895 99.358) (width 0.2) (layer "B.Cu") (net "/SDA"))
 (segment (start 142.46 100.42) (end 153.38 100.42) (width 0.2) (layer "B.Cu") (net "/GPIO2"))
 (segment (start 111.96 130.92) (end 142.46 100.42) (width 0.2) (layer "B.Cu") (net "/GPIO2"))
 (segment (start 154.442 104.022) (end 153.38 102.96) (width 0.2) (layer "B.Cu") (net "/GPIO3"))
 (segment (start 154.442 125.402) (end 154.442 104.022) (width 0.2) (layer "B.Cu") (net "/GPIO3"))
 (segment (start 159.96 130.92) (end 154.442 125.402) (width 0.2) (layer "B.Cu") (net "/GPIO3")))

